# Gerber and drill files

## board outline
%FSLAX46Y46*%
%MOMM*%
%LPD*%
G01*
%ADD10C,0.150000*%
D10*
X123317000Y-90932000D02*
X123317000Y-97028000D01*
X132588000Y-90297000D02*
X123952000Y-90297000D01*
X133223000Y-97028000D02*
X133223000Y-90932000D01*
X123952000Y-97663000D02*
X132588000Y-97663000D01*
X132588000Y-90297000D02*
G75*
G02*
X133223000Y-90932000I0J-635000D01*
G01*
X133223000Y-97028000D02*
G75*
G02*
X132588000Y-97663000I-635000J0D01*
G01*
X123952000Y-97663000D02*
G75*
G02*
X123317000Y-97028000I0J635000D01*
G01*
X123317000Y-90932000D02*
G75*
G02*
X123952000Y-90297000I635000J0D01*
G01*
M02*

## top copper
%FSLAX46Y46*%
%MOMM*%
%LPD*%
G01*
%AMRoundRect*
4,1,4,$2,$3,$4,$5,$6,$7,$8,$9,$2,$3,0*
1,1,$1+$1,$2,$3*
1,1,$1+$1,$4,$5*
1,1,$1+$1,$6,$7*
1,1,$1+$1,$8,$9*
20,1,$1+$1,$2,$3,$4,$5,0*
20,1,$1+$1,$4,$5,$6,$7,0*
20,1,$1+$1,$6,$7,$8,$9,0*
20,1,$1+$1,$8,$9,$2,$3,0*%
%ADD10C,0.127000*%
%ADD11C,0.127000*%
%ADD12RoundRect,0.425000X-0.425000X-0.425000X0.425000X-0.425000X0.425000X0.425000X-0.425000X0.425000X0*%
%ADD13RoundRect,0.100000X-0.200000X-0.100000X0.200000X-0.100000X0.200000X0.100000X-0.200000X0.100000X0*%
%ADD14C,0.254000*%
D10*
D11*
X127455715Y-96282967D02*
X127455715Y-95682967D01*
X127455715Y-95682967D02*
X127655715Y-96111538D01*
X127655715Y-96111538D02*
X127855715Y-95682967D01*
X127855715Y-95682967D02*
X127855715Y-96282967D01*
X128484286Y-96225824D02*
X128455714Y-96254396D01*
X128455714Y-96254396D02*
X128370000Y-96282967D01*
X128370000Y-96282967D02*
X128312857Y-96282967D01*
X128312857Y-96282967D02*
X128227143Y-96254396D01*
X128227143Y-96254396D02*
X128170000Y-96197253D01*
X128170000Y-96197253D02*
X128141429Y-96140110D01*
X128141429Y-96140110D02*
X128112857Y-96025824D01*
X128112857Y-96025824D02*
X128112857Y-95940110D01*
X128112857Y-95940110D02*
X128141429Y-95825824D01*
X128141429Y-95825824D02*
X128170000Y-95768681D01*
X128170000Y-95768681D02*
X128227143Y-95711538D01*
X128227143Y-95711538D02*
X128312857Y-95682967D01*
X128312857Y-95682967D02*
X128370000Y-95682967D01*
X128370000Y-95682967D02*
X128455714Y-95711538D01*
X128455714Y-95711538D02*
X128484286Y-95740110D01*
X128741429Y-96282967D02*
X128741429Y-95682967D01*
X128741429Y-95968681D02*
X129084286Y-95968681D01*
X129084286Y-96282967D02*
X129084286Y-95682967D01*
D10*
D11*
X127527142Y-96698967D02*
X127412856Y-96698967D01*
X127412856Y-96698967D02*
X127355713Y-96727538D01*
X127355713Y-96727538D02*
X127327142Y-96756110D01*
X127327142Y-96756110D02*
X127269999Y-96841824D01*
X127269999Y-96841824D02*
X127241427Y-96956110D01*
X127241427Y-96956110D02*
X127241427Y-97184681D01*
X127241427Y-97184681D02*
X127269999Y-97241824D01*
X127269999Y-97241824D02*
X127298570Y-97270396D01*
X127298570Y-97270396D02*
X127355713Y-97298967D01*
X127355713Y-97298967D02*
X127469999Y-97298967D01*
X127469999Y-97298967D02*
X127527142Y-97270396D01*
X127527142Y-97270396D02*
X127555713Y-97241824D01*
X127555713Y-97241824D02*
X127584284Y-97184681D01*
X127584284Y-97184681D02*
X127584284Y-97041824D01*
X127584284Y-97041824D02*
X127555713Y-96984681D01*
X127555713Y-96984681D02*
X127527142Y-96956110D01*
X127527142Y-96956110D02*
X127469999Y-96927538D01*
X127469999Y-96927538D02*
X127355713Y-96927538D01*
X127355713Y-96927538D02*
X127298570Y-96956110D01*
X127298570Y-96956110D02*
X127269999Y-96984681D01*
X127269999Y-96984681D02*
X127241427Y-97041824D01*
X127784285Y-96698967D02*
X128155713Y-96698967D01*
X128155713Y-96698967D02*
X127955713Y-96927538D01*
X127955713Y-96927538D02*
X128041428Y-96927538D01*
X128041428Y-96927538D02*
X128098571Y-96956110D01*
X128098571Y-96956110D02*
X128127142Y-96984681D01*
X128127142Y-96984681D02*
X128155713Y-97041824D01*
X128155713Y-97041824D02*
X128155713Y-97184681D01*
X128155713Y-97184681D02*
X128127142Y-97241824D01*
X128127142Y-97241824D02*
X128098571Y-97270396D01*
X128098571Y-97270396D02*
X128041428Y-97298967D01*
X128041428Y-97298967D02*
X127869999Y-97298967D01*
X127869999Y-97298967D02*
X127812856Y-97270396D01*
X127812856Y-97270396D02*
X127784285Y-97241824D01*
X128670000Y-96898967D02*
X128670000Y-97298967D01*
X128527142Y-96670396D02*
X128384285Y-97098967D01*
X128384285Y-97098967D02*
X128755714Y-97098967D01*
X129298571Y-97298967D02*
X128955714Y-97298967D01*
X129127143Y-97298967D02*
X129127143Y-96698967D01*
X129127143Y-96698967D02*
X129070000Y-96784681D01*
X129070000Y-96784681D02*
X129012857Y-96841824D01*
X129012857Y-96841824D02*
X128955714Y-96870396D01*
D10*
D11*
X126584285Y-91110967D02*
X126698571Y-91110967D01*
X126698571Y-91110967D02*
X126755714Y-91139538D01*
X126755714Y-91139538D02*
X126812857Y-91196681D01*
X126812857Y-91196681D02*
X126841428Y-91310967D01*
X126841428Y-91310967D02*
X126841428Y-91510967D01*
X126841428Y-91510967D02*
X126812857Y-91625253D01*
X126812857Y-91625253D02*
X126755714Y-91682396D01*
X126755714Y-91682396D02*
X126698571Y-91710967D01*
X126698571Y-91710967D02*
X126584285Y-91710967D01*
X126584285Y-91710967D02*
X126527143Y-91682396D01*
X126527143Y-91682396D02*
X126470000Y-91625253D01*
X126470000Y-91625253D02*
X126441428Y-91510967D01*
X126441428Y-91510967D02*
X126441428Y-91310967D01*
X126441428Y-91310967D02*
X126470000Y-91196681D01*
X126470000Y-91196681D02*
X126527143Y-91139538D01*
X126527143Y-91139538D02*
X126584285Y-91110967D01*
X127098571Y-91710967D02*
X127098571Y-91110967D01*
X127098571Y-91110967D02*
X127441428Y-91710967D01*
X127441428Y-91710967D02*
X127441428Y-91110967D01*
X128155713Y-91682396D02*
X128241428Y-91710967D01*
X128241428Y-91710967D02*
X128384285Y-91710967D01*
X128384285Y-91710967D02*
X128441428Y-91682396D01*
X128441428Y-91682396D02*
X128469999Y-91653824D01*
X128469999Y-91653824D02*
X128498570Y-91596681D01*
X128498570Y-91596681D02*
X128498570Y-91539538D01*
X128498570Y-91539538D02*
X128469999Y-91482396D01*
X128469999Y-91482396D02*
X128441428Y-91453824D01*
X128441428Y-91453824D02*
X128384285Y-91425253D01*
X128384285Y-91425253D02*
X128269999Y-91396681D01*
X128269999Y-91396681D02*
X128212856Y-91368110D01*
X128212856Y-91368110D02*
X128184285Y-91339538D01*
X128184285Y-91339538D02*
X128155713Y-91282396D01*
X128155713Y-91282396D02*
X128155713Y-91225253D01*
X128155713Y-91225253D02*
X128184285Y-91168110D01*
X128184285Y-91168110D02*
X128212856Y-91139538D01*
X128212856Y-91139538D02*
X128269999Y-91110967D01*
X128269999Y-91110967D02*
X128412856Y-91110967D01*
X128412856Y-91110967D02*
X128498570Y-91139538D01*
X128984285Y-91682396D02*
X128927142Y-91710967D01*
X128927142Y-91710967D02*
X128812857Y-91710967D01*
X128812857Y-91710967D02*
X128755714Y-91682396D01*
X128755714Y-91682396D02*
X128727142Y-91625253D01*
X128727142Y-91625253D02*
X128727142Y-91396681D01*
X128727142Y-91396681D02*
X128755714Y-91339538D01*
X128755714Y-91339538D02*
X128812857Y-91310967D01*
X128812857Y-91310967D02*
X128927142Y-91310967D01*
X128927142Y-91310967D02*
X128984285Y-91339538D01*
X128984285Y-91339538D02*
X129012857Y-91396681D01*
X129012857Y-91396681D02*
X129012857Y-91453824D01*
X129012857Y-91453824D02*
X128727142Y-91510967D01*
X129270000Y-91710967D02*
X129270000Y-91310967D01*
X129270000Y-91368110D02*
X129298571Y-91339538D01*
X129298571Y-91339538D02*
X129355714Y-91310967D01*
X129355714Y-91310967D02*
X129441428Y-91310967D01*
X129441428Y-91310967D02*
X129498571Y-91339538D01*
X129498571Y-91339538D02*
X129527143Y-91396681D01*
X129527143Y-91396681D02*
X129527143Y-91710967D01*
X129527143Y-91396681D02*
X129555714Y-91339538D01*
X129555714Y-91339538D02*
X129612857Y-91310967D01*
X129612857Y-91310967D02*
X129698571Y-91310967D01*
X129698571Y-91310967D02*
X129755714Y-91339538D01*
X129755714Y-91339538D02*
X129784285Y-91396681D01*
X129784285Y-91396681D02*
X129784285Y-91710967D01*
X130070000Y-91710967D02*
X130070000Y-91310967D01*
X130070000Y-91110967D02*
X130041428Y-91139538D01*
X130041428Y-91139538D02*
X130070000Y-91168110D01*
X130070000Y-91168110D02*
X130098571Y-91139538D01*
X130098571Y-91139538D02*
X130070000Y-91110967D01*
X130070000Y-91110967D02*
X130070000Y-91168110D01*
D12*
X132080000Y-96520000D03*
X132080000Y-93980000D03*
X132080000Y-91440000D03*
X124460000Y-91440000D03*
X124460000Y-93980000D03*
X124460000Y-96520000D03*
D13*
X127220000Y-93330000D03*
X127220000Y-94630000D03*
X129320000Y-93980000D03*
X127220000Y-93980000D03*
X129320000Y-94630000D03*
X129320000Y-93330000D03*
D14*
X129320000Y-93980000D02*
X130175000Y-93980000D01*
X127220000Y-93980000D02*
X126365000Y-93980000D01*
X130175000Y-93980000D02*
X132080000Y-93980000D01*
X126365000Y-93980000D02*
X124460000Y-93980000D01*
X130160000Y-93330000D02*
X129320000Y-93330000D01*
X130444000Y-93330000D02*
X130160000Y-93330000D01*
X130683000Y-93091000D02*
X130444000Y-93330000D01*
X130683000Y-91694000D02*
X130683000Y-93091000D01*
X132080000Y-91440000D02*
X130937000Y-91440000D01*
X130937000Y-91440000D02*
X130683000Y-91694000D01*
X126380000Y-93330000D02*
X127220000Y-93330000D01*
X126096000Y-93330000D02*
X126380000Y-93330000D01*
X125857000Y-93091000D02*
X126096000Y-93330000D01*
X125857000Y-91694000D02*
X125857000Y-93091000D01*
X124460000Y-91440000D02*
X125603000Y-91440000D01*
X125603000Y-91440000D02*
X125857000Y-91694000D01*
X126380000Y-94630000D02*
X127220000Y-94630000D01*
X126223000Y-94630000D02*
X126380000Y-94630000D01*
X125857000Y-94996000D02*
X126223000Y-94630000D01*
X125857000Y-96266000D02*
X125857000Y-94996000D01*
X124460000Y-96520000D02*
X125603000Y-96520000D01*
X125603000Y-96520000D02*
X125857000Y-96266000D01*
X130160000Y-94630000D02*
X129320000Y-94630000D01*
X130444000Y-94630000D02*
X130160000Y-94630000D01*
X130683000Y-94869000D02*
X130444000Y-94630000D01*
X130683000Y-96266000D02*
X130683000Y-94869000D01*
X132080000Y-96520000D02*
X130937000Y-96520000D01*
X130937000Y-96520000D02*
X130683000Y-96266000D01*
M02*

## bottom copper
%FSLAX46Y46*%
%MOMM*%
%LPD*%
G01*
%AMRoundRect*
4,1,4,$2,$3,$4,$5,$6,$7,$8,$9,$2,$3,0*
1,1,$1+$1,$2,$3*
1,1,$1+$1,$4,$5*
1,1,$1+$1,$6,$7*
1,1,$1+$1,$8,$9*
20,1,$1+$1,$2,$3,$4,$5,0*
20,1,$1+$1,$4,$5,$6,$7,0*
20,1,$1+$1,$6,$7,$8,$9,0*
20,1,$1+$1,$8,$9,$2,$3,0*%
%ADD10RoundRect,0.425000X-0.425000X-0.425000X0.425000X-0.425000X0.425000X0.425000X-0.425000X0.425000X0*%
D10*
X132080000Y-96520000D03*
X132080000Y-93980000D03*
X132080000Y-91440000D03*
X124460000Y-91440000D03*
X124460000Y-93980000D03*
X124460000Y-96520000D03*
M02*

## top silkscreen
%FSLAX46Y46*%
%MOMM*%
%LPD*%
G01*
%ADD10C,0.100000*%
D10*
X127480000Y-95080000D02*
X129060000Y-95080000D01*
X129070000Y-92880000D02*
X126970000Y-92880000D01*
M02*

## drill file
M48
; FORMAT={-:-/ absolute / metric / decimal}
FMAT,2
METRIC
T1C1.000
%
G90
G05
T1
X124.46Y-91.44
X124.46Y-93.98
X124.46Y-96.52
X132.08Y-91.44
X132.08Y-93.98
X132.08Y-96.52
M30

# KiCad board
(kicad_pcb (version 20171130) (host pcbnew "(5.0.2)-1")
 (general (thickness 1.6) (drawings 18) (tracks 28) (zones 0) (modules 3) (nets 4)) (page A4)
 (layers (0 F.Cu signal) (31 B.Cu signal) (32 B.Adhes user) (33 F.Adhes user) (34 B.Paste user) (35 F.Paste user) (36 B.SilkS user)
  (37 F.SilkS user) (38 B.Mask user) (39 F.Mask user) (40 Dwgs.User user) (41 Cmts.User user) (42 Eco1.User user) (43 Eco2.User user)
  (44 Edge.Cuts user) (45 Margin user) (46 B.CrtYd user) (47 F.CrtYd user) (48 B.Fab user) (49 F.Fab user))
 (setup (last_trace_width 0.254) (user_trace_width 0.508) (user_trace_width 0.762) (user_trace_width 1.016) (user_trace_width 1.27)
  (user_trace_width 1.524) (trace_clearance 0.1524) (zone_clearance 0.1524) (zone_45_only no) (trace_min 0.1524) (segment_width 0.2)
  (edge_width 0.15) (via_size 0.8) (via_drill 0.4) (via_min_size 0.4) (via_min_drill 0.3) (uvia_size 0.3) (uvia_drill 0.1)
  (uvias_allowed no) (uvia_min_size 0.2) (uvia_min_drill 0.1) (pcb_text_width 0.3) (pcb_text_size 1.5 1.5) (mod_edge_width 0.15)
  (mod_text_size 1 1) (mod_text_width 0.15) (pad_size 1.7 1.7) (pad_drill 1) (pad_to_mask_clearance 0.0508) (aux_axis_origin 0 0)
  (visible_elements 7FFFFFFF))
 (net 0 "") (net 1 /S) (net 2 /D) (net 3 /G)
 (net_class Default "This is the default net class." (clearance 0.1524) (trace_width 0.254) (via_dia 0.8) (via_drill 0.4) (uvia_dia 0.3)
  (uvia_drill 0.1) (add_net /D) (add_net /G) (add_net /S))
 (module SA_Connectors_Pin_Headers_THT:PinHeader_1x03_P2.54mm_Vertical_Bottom (layer F.Cu) (at 132.08 91.44)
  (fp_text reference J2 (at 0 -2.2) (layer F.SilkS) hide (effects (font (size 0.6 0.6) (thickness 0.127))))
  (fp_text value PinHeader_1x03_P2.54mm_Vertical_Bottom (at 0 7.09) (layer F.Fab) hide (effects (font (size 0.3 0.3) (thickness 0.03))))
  (pad 3 thru_hole roundrect (at 0 5.08) (size 1.7 1.7) (drill 1) (layers *.Cu *.Mask) (roundrect_rratio 0.25) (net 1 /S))
  (pad 2 thru_hole roundrect (at 0 2.54) (size 1.7 1.7) (drill 1) (layers *.Cu *.Mask) (roundrect_rratio 0.25) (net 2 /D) (zone_connect 2))
  (pad 1 thru_hole roundrect (at 0 0) (size 1.7 1.7) (drill 1) (layers *.Cu *.Mask) (roundrect_rratio 0.25) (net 2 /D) (zone_connect 2)))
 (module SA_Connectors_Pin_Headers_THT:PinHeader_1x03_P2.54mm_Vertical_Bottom (layer F.Cu) (at 124.46 91.44)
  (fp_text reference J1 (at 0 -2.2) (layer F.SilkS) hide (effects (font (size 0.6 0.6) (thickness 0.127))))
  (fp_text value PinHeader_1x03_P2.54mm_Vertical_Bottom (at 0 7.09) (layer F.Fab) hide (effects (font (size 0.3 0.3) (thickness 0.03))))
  (pad 1 thru_hole roundrect (at 0 0) (size 1.7 1.7) (drill 1) (layers *.Cu *.Mask) (roundrect_rratio 0.25) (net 2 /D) (zone_connect 2))
  (pad 2 thru_hole roundrect (at 0 2.54) (size 1.7 1.7) (drill 1) (layers *.Cu *.Mask) (roundrect_rratio 0.25) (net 2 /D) (zone_connect 2))
  (pad 3 thru_hole roundrect (at 0 5.08) (size 1.7 1.7) (drill 1) (layers *.Cu *.Mask) (roundrect_rratio 0.25) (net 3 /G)))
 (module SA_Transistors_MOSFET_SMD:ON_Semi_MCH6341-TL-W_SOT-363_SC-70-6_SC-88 (layer F.Cu) (at 128.27 93.98)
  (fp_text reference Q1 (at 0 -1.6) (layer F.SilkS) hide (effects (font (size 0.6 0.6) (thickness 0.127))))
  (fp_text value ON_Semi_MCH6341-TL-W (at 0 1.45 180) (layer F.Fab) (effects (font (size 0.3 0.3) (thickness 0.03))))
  (fp_line (start -0.79 1.1) (end 0.79 1.1) (layer F.SilkS) (width 0.1))
  (fp_line (start 0.8 -1.1) (end -1.3 -1.1) (layer F.SilkS) (width 0.1))
  (pad D smd roundrect (at -1.05 -0.65) (size 0.6 0.4) (layers F.Cu F.Paste F.Mask) (roundrect_rratio 0.25) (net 2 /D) (zone_connect 2))
  (pad G smd roundrect (at -1.05 0.65) (size 0.6 0.4) (layers F.Cu F.Paste F.Mask) (roundrect_rratio 0.25) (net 3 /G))
  (pad D smd roundrect (at 1.05 0) (size 0.6 0.4) (layers F.Cu F.Paste F.Mask) (roundrect_rratio 0.25) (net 2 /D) (zone_connect 2))
  (pad D smd roundrect (at -1.05 0) (size 0.6 0.4) (layers F.Cu F.Paste F.Mask) (roundrect_rratio 0.25) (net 2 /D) (zone_connect 2))
  (pad S smd roundrect (at 1.05 0.65) (size 0.6 0.4) (layers F.Cu F.Paste F.Mask) (roundrect_rratio 0.25) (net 1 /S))
  (pad D smd roundrect (at 1.05 -0.65) (size 0.6 0.4) (layers F.Cu F.Paste F.Mask) (roundrect_rratio 0.25) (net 2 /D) (zone_connect 2)))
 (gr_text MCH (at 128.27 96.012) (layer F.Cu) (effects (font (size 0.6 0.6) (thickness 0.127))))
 (gr_line (start 123.317 90.932) (end 123.317 97.028) (layer Edge.Cuts) (width 0.15))
 (gr_line (start 132.588 90.297) (end 123.952 90.297) (layer Edge.Cuts) (width 0.15))
 (gr_line (start 133.223 97.028) (end 133.223 90.932) (layer Edge.Cuts) (width 0.15))
 (gr_line (start 123.952 97.663) (end 132.588 97.663) (layer Edge.Cuts) (width 0.15))
 (gr_arc (start 132.588 90.932) (end 133.223 90.932) (angle -90) (layer Edge.Cuts) (width 0.15))
 (gr_arc (start 132.588 97.028) (end 132.588 97.663) (angle -90) (layer Edge.Cuts) (width 0.15))
 (gr_arc (start 123.952 97.028) (end 123.317 97.028) (angle -90) (layer Edge.Cuts) (width 0.15))
 (gr_arc (start 123.952 90.932) (end 123.952 90.297) (angle -90) (layer Edge.Cuts) (width 0.15))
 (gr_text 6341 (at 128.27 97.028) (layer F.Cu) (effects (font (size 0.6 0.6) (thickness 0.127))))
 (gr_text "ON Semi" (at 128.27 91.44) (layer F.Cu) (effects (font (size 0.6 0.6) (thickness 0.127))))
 (segment (start 129.32 93.98) (end 130.175 93.98) (width 0.254) (layer F.Cu) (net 2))
 (segment (start 127.22 93.98) (end 126.365 93.98) (width 0.254) (layer F.Cu) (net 2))
 (segment (start 130.175 93.98) (end 132.08 93.98) (width 0.254) (layer F.Cu) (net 2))
 (segment (start 126.365 93.98) (end 124.46 93.98) (width 0.254) (layer F.Cu) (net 2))
 (segment (start 130.16 93.33) (end 129.32 93.33) (width 0.254) (layer F.Cu) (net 2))
 (segment (start 130.444 93.33) (end 130.16 93.33) (width 0.254) (layer F.Cu) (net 2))
 (segment (start 130.683 93.091) (end 130.444 93.33) (width 0.254) (layer F.Cu) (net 2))
 (segment (start 130.683 91.694) (end 130.683 93.091) (width 0.254) (layer F.Cu) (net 2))
 (segment (start 132.08 91.44) (end 130.937 91.44) (width 0.254) (layer F.Cu) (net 2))
 (segment (start 130.937 91.44) (end 130.683 91.694) (width 0.254) (layer F.Cu) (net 2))
 (segment (start 126.38 93.33) (end 127.22 93.33) (width 0.254) (layer F.Cu) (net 2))
 (segment (start 126.096 93.33) (end 126.38 93.33) (width 0.254) (layer F.Cu) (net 2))
 (segment (start 125.857 93.091) (end 126.096 93.33) (width 0.254) (layer F.Cu) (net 2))
 (segment (start 125.857 91.694) (end 125.857 93.091) (width 0.254) (layer F.Cu) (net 2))
 (segment (start 124.46 91.44) (end 125.603 91.44) (width 0.254) (layer F.Cu) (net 2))
 (segment (start 125.603 91.44) (end 125.857 91.694) (width 0.254) (layer F.Cu) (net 2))
 (segment (start 126.38 94.63) (end 127.22 94.63) (width 0.254) (layer F.Cu) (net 3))
 (segment (start 126.223 94.63) (end 126.38 94.63) (width 0.254) (layer F.Cu) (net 3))
 (segment (start 125.857 94.996) (end 126.223 94.63) (width 0.254) (layer F.Cu) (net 3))
 (segment (start 125.857 96.266) (end 125.857 94.996) (width 0.254) (layer F.Cu) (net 3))
 (segment (start 124.46 96.52) (end 125.603 96.52) (width 0.254) (layer F.Cu) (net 3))
 (segment (start 125.603 96.52) (end 125.857 96.266) (width 0.254) (layer F.Cu) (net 3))
 (segment (start 130.16 94.63) (end 129.32 94.63) (width 0.254) (layer F.Cu) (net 1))
 (segment (start 130.444 94.63) (end 130.16 94.63) (width 0.254) (layer F.Cu) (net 1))
 (segment (start 130.683 94.869) (end 130.444 94.63) (width 0.254) (layer F.Cu) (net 1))
 (segment (start 130.683 96.266) (end 130.683 94.869) (width 0.254) (layer F.Cu) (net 1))
 (segment (start 132.08 96.52) (end 130.937 96.52) (width 0.254) (layer F.Cu) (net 1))
 (segment (start 130.937 96.52) (end 130.683 96.266) (width 0.254) (layer F.Cu) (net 1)))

